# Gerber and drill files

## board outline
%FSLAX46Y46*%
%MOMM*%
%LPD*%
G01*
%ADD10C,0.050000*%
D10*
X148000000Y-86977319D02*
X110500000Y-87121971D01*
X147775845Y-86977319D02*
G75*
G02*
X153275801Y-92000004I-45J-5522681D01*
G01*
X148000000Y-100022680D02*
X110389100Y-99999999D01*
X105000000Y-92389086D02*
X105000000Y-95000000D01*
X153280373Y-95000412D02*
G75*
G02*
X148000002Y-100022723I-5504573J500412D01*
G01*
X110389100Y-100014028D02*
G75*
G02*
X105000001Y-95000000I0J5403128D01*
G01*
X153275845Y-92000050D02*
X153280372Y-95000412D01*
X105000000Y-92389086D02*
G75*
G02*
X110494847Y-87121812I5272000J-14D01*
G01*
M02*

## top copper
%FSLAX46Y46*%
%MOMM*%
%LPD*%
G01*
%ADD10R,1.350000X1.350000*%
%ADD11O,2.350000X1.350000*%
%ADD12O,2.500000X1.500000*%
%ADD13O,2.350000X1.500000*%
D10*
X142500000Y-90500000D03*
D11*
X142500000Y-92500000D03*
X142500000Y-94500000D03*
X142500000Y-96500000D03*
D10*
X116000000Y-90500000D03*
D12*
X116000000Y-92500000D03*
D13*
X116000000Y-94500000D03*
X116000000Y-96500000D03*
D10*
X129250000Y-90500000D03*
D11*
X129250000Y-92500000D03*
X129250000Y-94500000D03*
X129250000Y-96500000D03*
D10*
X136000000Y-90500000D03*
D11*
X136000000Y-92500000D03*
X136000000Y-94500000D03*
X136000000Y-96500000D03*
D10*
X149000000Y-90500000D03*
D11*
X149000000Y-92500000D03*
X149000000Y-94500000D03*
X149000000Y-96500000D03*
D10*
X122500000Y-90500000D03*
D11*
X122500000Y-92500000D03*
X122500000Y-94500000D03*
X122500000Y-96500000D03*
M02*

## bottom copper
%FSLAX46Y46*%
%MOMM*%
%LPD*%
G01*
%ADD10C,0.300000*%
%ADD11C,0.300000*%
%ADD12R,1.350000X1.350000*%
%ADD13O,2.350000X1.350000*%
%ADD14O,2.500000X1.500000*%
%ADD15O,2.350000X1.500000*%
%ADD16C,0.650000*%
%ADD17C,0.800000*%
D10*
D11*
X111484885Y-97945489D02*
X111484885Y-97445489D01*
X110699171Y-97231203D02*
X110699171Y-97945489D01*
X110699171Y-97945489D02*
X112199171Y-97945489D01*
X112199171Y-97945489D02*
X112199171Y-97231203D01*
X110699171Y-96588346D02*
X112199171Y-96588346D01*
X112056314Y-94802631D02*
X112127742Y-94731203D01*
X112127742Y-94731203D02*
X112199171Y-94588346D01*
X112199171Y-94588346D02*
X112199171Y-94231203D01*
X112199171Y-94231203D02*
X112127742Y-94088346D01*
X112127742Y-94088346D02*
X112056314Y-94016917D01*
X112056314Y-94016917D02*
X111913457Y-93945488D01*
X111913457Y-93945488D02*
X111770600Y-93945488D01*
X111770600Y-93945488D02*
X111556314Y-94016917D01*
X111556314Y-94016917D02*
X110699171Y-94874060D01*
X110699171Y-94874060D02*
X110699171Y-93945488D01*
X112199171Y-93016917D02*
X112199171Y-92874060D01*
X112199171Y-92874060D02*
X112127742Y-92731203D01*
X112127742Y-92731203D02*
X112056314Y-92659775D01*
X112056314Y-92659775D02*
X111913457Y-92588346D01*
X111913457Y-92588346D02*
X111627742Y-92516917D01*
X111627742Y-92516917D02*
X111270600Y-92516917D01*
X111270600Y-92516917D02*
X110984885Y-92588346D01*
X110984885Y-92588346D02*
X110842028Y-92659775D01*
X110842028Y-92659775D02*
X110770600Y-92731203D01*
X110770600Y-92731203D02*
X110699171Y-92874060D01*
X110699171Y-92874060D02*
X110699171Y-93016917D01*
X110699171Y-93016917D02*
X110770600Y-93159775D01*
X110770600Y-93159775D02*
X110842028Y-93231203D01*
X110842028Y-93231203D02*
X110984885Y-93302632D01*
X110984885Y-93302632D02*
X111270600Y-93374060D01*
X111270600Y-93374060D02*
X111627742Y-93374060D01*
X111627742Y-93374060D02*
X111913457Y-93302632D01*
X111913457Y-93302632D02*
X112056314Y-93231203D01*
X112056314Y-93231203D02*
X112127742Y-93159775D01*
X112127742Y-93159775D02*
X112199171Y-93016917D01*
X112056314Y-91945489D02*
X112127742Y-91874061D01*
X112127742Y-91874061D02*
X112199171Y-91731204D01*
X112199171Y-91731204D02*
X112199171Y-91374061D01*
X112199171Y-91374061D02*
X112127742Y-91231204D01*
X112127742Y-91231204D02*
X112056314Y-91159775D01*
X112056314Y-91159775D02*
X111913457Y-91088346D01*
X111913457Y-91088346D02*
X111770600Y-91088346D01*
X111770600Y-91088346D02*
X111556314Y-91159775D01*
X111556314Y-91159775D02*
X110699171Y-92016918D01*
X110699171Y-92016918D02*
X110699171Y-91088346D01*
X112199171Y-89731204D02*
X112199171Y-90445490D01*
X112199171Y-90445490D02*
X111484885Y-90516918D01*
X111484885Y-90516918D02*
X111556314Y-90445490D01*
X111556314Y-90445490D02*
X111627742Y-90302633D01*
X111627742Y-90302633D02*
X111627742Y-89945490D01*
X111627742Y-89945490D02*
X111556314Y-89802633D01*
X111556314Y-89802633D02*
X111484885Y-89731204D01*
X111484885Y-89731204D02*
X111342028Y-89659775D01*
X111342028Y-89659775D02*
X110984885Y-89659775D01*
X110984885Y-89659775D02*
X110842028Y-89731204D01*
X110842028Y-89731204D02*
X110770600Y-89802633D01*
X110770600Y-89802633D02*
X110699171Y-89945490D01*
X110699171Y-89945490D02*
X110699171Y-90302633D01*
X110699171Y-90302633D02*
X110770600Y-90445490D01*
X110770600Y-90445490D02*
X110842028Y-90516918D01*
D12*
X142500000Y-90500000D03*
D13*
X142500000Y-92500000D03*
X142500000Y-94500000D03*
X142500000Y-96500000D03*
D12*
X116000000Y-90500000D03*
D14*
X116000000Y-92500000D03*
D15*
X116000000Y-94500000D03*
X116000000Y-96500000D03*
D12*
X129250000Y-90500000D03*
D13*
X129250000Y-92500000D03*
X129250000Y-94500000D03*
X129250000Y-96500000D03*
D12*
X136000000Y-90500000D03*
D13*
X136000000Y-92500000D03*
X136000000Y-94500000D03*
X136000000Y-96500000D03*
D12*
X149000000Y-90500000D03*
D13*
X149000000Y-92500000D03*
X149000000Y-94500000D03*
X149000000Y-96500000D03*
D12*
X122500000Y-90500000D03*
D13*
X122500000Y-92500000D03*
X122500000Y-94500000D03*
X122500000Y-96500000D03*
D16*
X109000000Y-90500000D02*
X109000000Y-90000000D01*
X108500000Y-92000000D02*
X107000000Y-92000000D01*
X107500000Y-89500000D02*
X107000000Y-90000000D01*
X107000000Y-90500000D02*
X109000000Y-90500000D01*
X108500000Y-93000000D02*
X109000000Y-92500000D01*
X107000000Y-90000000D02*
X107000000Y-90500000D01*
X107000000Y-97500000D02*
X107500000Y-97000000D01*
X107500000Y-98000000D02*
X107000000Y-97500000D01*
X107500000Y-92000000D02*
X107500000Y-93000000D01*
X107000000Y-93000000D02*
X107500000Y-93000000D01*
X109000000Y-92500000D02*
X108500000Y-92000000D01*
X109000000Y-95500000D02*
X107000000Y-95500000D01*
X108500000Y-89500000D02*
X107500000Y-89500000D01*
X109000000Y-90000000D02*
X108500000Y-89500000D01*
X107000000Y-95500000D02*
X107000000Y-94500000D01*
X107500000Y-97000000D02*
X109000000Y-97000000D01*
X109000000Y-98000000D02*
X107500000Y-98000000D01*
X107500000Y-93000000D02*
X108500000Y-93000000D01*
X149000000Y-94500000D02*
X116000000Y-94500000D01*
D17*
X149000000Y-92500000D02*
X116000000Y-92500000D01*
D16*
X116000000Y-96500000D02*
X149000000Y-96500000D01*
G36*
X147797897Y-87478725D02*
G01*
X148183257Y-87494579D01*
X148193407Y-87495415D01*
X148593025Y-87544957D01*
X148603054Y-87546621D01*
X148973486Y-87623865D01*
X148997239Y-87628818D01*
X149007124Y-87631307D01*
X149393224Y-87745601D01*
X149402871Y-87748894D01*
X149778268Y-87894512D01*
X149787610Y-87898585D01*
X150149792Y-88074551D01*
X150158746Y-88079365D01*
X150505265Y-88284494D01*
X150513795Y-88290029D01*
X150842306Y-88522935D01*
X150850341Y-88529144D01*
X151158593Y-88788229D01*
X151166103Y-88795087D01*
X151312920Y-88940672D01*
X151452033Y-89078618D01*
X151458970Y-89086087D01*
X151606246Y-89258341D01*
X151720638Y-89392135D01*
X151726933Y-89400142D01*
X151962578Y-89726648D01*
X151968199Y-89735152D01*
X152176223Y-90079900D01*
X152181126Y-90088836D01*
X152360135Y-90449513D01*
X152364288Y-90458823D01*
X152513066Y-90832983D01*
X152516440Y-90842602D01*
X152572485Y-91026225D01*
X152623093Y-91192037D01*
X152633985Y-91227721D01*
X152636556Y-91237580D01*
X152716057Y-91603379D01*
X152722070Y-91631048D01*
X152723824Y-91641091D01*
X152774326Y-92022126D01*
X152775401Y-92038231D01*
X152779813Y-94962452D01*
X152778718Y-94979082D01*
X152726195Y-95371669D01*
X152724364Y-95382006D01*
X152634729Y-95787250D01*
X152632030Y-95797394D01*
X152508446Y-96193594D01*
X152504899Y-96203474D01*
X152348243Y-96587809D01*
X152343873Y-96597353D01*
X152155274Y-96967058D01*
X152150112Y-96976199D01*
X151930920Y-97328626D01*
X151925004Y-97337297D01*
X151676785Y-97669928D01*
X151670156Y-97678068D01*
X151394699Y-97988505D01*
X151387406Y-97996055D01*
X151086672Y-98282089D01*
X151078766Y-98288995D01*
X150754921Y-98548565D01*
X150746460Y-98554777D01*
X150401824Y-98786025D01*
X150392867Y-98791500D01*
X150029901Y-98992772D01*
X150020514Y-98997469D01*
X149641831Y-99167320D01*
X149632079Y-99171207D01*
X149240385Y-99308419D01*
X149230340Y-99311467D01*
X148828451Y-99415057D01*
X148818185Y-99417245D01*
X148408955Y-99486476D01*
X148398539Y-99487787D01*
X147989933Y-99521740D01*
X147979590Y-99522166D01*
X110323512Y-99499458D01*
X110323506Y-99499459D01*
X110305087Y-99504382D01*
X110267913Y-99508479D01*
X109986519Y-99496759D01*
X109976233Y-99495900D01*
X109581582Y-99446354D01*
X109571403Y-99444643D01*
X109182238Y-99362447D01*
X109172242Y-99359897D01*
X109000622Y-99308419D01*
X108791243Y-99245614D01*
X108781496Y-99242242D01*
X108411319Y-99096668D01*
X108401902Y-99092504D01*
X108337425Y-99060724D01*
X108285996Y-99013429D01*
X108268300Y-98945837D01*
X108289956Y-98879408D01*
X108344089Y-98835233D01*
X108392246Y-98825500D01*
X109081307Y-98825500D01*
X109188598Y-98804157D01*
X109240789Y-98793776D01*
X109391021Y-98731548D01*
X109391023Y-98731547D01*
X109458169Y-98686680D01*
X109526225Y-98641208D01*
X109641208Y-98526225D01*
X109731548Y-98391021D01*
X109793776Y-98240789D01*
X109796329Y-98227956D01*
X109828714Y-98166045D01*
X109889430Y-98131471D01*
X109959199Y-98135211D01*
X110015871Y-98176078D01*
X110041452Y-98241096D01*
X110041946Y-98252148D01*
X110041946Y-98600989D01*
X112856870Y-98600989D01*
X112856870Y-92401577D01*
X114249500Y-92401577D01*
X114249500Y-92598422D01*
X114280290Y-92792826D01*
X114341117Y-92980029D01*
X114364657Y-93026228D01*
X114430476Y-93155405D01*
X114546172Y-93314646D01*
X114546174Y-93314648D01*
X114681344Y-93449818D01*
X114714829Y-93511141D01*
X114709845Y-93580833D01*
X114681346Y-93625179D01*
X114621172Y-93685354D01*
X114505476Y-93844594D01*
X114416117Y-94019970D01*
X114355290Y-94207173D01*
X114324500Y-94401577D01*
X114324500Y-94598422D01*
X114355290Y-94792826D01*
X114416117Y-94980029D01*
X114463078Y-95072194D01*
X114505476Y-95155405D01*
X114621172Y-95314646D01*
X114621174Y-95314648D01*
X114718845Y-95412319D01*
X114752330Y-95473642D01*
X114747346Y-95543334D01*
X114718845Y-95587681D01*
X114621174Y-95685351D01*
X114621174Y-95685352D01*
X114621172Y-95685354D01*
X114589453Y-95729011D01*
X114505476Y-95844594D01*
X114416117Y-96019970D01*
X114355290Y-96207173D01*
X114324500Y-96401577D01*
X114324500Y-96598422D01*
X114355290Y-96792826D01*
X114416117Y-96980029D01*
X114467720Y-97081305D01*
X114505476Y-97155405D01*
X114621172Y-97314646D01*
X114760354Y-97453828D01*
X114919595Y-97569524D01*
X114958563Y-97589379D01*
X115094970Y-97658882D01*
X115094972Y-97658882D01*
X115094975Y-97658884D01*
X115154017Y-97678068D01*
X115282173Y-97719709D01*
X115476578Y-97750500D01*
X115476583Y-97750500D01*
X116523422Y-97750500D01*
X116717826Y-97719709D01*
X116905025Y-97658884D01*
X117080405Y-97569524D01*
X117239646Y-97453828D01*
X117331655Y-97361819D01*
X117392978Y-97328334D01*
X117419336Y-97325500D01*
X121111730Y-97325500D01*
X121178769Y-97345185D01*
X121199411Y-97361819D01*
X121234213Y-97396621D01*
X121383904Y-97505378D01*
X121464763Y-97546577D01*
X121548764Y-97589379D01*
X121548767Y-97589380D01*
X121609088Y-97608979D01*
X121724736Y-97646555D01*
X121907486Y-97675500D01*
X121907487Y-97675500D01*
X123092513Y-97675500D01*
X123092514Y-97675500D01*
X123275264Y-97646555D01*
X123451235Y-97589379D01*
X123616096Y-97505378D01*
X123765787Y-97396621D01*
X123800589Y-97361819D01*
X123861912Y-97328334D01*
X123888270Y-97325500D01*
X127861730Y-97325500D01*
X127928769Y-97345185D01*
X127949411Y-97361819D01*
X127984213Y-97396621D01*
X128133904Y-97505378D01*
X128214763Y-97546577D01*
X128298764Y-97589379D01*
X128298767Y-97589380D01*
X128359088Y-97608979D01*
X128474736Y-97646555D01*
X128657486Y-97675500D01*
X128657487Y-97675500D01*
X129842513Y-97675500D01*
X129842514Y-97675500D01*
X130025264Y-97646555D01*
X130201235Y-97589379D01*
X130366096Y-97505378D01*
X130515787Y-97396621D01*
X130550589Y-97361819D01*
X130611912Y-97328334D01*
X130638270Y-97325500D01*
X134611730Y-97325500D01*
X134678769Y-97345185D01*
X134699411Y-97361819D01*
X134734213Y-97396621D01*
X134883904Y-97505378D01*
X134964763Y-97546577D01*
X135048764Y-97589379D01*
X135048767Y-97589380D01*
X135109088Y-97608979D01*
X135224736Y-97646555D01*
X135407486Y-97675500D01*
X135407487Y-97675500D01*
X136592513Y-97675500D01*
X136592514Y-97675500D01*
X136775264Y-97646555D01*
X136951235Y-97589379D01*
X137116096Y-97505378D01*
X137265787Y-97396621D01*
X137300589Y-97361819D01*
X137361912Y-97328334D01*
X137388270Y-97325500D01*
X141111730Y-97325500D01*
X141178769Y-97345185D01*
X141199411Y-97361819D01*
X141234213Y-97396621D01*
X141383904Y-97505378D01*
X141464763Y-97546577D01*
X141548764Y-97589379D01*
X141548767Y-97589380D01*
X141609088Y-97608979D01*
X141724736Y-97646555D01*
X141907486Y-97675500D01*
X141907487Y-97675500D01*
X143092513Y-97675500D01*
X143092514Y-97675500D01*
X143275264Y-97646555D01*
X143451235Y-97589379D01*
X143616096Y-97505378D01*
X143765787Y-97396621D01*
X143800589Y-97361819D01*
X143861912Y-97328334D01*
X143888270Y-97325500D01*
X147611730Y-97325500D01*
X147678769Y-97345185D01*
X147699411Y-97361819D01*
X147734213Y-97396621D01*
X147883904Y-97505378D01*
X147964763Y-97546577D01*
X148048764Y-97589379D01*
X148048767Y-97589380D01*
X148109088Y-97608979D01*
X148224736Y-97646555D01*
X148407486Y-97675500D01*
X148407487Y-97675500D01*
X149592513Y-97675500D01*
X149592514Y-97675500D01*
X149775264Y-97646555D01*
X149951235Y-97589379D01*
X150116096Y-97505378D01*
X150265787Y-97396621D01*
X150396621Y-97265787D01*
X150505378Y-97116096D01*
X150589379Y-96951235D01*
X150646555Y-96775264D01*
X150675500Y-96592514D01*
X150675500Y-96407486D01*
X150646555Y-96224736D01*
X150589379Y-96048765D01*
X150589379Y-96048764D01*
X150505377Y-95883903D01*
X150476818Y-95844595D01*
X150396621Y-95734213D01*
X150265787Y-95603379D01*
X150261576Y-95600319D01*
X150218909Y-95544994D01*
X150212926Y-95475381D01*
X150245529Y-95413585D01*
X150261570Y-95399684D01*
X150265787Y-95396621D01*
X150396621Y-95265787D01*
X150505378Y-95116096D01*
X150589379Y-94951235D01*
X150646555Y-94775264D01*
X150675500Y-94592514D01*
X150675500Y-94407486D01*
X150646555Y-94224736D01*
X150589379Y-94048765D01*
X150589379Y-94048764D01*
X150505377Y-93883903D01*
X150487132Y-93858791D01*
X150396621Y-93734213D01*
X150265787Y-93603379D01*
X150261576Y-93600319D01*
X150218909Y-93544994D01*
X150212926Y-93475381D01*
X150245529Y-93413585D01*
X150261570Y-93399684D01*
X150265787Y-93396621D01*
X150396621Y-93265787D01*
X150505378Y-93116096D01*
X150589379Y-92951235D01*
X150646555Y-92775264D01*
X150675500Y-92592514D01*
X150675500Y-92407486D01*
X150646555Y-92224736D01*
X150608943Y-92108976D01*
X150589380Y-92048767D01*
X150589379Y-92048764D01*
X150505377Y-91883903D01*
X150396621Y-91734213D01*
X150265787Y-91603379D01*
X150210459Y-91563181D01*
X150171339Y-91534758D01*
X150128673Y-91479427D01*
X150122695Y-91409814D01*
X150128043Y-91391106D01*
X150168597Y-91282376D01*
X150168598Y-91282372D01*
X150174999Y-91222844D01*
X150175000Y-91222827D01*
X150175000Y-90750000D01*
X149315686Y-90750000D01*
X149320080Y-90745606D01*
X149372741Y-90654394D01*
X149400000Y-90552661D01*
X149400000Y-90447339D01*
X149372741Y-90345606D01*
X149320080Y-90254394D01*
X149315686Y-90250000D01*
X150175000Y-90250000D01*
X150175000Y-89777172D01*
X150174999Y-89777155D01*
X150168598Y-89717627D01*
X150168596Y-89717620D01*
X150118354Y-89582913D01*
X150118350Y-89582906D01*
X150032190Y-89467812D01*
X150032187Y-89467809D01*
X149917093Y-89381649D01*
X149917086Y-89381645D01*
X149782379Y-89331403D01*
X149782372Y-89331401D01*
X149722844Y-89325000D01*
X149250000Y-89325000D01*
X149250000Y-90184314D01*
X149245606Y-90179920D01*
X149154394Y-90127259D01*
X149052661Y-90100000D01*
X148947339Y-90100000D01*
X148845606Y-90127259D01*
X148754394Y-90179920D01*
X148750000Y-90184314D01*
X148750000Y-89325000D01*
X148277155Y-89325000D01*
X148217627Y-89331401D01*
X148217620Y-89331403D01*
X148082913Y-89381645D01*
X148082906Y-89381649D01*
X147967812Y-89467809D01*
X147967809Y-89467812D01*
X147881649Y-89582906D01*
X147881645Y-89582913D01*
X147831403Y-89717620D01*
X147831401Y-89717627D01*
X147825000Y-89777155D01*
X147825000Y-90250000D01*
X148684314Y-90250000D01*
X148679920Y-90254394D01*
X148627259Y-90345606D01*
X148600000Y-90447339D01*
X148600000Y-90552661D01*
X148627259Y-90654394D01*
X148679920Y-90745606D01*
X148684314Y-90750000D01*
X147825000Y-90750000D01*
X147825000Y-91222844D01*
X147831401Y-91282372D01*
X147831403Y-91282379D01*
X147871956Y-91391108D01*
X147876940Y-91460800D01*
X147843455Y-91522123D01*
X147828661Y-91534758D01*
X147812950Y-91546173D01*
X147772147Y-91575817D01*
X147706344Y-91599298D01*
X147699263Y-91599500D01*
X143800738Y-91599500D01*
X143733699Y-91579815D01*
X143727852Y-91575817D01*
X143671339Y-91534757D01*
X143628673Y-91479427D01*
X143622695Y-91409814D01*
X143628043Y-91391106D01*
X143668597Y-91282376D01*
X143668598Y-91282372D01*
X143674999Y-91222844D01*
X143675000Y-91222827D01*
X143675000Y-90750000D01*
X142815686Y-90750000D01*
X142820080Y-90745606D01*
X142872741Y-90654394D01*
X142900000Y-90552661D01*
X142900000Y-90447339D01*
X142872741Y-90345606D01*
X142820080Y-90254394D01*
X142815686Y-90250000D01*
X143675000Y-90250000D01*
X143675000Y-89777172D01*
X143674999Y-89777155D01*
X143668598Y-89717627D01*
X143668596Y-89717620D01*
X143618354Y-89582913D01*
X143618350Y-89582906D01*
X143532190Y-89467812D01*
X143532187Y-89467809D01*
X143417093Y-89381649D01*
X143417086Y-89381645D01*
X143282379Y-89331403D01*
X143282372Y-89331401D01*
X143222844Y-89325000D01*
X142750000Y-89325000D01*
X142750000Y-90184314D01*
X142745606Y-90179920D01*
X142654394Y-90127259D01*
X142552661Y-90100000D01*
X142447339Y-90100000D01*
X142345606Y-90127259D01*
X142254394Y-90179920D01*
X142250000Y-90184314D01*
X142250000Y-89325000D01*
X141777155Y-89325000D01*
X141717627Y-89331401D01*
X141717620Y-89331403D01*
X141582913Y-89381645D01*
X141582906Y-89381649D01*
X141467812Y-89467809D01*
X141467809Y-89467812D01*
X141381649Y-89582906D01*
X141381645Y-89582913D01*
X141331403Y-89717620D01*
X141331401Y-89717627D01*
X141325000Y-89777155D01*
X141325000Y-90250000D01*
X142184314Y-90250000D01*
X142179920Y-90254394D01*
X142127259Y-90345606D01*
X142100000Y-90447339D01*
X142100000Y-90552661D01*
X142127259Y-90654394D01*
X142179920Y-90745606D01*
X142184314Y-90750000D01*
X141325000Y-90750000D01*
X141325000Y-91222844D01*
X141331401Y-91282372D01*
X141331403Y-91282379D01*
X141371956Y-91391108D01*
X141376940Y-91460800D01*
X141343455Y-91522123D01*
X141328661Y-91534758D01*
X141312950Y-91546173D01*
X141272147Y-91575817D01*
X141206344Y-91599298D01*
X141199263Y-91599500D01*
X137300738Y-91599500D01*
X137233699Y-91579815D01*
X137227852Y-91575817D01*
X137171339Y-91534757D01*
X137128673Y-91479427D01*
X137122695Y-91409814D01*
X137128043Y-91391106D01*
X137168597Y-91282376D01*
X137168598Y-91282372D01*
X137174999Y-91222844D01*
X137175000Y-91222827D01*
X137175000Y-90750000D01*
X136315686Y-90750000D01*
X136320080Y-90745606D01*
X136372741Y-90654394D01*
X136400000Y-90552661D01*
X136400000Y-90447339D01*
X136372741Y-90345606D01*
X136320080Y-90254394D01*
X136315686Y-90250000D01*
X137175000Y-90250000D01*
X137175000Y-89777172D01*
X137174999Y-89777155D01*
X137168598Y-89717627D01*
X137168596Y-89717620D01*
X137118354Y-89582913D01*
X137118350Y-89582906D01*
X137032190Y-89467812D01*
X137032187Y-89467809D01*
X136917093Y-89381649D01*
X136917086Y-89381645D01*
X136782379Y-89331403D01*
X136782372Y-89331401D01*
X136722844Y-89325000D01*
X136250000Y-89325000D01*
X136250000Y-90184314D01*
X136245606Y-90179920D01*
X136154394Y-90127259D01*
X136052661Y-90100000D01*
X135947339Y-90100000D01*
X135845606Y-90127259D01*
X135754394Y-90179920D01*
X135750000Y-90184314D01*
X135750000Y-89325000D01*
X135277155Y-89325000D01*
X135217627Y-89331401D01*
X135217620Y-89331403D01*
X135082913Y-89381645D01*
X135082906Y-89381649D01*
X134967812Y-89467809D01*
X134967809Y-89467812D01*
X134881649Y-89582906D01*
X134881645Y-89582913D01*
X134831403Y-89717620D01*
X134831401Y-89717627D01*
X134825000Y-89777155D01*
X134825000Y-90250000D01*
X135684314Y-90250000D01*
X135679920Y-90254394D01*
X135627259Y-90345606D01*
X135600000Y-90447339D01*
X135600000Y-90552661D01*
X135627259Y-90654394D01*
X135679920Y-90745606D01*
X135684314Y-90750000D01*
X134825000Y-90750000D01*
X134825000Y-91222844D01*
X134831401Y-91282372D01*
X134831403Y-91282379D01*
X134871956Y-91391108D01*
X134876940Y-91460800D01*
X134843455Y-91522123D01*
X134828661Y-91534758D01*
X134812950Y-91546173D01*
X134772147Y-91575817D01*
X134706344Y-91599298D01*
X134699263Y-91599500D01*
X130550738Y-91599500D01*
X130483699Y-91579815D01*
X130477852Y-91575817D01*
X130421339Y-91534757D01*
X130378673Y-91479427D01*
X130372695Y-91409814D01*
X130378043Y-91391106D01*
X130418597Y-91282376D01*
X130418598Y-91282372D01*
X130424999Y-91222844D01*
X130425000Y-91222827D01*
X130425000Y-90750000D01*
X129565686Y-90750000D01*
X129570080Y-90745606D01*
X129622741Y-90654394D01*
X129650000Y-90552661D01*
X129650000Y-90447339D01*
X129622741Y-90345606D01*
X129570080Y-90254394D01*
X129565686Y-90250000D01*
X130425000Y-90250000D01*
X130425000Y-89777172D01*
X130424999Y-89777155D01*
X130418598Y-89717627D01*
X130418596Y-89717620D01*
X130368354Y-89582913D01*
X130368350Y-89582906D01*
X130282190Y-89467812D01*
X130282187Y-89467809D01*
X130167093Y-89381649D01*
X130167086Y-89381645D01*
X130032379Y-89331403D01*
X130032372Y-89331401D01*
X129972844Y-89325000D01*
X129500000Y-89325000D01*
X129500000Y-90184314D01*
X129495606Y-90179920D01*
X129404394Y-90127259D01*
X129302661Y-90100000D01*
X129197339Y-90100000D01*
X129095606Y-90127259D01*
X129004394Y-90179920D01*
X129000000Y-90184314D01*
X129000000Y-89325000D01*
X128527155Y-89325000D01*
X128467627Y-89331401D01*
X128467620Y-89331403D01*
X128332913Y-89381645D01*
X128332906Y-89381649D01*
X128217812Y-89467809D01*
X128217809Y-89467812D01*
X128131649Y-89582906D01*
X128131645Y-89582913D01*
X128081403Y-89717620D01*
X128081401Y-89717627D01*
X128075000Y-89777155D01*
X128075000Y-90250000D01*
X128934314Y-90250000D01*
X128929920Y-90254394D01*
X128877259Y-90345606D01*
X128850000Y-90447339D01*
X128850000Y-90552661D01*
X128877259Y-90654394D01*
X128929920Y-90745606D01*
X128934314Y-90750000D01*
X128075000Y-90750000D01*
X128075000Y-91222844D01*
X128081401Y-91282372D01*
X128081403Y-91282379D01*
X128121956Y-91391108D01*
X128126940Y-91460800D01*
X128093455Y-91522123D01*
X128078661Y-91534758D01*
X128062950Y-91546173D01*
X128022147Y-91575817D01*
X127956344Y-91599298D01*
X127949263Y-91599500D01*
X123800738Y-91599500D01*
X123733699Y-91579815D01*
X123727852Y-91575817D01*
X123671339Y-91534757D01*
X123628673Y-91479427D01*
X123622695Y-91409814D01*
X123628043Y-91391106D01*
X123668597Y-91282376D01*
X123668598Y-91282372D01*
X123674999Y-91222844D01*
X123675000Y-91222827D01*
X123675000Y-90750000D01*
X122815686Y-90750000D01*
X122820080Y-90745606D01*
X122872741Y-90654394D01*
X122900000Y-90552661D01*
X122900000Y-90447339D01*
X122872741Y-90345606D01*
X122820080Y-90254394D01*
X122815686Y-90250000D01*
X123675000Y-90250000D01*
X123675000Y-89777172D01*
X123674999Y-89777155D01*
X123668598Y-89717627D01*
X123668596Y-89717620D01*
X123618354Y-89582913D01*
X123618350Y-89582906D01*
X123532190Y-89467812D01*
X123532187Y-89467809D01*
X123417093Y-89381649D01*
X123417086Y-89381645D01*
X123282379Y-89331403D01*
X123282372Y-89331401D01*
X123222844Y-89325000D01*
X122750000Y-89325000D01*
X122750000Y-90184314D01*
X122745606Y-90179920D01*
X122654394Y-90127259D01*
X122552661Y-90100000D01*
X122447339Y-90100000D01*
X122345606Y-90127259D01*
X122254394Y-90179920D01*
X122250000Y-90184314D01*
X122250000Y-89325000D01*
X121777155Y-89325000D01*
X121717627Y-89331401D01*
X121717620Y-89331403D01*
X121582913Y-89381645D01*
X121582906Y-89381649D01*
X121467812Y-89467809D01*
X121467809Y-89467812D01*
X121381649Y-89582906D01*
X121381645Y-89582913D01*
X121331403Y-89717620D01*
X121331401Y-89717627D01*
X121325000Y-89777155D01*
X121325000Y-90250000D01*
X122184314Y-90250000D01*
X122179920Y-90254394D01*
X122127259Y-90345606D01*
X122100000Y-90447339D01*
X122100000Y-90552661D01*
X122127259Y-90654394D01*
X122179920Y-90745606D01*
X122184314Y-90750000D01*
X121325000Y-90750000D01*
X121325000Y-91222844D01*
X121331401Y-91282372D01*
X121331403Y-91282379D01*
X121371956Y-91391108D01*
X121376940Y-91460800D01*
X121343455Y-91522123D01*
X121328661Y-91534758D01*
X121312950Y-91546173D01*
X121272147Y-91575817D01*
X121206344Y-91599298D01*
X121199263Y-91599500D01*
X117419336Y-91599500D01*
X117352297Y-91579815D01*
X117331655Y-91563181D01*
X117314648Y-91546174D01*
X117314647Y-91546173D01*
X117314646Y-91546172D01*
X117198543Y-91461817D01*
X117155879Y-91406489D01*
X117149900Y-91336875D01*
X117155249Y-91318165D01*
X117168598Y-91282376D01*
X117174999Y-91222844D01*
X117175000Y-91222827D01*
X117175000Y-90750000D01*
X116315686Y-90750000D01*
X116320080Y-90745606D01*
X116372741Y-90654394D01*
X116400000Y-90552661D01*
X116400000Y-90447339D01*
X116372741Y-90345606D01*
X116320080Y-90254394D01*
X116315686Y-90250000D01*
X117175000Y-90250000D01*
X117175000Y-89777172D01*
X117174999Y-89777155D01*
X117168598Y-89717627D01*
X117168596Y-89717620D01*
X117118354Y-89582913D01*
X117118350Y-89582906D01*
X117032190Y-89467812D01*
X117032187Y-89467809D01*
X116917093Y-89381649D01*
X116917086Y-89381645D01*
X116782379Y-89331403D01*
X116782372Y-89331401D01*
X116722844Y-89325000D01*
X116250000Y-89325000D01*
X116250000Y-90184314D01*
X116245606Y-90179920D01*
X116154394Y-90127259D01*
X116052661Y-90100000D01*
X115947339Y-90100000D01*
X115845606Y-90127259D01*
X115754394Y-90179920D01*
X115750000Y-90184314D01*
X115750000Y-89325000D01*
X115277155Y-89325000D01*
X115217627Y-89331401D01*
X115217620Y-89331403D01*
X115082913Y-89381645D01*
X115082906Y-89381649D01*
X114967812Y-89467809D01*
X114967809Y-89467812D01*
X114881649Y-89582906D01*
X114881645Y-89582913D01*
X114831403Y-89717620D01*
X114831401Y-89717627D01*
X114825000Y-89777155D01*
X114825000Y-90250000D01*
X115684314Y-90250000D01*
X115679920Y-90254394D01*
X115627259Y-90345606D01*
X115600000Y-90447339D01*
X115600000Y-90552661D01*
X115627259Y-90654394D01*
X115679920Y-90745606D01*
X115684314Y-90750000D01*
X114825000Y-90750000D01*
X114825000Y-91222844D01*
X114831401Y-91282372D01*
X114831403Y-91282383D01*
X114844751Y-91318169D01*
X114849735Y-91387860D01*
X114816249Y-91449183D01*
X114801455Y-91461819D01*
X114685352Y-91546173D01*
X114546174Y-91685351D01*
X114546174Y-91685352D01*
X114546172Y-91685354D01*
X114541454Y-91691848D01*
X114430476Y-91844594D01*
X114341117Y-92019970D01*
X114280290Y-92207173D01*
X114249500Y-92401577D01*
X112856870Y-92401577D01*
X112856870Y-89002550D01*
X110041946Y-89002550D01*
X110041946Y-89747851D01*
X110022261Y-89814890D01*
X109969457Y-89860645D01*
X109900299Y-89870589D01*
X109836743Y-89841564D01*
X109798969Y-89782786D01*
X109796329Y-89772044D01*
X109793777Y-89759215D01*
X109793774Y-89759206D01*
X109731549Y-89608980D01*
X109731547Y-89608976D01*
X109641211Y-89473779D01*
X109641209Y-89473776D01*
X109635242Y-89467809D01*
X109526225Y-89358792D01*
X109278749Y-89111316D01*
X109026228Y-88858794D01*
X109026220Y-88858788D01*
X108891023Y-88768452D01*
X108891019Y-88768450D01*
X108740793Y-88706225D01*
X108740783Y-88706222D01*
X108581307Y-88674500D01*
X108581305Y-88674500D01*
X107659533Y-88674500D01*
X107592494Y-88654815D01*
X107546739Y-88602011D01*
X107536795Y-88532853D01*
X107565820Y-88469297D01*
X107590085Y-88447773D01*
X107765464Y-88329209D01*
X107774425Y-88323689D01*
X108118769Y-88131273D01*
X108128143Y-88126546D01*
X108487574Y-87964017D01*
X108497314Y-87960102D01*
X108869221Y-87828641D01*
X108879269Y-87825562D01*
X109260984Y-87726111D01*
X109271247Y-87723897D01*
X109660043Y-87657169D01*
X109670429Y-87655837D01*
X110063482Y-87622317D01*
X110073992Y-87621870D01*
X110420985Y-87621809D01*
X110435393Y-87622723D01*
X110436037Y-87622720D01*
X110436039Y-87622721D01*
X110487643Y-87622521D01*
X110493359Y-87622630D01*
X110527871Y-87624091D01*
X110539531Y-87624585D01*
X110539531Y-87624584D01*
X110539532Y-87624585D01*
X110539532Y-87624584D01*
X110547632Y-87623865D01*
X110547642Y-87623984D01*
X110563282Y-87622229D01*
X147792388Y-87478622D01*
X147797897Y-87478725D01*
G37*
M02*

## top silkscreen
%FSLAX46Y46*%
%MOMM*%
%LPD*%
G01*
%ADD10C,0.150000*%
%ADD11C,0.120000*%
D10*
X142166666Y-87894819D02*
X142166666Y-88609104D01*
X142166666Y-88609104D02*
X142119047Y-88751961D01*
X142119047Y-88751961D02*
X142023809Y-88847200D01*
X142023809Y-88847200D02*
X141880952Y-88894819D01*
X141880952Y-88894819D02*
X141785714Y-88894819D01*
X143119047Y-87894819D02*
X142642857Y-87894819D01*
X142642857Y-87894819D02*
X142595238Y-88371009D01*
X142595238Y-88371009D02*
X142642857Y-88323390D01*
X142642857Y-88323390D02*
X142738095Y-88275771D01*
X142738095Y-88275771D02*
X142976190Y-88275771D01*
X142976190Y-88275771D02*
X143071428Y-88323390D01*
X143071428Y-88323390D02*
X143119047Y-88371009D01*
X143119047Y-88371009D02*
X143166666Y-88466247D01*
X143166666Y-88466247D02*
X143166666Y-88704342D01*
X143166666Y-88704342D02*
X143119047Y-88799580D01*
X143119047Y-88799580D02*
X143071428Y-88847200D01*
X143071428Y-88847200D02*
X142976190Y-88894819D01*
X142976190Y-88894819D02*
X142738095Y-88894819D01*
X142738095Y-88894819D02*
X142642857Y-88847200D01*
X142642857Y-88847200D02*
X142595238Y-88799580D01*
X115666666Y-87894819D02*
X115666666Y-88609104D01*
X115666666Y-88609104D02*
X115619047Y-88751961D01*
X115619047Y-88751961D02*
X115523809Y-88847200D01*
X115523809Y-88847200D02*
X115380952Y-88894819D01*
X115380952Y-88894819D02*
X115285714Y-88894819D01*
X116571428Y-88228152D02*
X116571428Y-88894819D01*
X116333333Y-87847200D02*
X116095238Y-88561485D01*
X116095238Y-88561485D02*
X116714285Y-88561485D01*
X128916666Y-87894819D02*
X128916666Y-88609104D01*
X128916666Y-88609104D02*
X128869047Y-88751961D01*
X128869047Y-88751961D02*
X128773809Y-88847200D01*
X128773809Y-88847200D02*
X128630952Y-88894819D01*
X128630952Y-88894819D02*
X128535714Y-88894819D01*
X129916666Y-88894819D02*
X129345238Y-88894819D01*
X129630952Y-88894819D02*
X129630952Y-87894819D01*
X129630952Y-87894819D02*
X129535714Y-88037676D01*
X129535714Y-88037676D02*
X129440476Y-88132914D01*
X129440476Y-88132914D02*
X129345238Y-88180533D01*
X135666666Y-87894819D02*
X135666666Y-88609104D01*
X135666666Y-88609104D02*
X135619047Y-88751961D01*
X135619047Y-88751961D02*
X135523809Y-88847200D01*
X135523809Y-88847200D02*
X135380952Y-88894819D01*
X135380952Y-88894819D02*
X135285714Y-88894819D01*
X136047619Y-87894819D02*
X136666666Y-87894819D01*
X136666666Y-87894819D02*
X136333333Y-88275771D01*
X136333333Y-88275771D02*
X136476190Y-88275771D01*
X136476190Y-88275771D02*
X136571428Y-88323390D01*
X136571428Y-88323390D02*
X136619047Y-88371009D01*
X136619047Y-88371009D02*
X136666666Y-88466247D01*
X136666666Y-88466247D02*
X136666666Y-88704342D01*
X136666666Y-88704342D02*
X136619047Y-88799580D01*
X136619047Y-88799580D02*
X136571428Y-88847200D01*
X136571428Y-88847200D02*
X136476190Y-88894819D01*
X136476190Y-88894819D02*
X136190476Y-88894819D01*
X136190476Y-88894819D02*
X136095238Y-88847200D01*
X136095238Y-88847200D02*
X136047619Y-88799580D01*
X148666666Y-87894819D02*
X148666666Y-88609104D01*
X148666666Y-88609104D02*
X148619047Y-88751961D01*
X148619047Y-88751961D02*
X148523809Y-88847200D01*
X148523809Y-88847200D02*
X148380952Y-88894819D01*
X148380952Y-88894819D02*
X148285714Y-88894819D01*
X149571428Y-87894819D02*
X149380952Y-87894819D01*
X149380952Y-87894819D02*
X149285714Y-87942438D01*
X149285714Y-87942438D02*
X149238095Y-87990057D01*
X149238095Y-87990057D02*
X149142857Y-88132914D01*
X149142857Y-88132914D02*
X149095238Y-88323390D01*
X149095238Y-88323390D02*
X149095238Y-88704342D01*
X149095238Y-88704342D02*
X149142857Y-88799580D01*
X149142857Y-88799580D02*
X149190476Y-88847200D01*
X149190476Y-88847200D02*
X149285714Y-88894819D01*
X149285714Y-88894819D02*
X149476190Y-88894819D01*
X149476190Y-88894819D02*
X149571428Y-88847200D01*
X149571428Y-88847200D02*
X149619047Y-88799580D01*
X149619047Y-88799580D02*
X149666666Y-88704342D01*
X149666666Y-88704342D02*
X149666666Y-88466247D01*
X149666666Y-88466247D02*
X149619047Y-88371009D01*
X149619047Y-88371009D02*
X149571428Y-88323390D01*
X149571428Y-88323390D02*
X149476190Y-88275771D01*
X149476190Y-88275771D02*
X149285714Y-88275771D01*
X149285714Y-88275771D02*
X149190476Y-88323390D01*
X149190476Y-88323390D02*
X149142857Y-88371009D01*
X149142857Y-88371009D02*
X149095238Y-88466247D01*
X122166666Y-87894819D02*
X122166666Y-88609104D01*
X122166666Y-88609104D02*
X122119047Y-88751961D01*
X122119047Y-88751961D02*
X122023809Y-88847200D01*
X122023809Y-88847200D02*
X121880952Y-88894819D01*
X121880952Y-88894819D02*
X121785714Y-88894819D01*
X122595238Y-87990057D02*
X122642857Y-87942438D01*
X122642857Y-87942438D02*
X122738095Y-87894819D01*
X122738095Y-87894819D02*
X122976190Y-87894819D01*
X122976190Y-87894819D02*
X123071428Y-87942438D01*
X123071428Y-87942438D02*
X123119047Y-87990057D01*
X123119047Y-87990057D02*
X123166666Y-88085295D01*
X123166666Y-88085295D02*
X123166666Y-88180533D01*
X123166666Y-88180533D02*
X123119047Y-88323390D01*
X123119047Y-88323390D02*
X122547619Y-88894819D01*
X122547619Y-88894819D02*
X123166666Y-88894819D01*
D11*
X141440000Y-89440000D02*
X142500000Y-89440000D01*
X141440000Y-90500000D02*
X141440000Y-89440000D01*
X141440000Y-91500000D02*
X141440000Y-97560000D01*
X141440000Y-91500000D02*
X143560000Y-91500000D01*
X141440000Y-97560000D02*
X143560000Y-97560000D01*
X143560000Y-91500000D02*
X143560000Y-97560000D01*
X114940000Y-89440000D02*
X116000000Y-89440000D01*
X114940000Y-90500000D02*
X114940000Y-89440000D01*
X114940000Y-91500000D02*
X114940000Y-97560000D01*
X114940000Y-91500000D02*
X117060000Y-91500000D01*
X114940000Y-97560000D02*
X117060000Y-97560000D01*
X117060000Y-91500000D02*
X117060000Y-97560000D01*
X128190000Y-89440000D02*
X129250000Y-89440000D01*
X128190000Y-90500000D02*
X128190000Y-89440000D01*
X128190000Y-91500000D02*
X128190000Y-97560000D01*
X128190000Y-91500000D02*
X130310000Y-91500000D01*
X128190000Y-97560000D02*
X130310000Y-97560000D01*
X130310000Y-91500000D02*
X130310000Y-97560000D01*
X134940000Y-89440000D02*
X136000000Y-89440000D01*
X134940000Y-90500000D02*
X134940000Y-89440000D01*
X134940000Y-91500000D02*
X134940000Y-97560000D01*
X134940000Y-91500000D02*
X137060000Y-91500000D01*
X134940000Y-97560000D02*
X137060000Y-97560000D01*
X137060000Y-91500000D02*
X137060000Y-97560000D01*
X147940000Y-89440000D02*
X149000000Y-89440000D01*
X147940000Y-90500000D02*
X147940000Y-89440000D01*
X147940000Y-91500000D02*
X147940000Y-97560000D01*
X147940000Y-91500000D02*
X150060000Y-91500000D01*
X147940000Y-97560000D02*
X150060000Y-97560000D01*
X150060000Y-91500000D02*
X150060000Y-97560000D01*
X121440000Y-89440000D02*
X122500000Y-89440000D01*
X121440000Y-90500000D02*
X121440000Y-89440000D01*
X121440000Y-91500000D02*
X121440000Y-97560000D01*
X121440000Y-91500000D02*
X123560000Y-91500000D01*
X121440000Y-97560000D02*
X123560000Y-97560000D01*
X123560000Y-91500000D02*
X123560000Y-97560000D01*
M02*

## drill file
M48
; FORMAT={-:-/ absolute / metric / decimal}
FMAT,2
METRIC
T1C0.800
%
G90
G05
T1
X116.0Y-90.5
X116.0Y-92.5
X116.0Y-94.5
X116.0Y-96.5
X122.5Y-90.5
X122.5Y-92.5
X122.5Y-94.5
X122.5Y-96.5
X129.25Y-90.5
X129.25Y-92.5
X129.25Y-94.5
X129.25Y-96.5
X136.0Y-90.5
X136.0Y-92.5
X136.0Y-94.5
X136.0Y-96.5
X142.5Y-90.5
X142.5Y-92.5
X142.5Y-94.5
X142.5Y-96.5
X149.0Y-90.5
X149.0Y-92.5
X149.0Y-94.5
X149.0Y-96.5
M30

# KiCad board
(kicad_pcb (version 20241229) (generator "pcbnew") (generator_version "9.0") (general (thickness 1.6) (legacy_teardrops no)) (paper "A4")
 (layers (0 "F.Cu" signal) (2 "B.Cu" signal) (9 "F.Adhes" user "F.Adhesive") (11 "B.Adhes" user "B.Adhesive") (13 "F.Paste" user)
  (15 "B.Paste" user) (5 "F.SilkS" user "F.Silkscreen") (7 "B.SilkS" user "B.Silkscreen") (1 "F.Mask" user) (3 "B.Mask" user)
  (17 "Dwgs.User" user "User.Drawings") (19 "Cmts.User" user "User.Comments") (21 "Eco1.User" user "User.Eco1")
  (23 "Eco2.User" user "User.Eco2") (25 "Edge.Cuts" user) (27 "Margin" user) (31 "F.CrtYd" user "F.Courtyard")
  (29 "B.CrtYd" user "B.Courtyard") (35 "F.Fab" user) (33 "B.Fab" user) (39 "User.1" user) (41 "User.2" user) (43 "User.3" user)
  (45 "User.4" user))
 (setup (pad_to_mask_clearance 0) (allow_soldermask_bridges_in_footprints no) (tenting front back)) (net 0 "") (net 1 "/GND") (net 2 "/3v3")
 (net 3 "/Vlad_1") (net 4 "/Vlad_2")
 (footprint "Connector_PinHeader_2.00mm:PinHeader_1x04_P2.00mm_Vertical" (layer "F.Cu") (at 142.5 90.5)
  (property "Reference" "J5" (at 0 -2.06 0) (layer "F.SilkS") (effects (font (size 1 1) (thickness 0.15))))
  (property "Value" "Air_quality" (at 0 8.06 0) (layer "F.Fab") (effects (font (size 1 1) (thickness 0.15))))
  (fp_line (start -1.06 -1.06) (end 0 -1.06) (stroke (width 0.12) (type solid)) (layer "F.SilkS"))
  (fp_line (start -1.06 0) (end -1.06 -1.06) (stroke (width 0.12) (type solid)) (layer "F.SilkS"))
  (fp_line (start -1.06 1) (end -1.06 7.06) (stroke (width 0.12) (type solid)) (layer "F.SilkS"))
  (fp_line (start -1.06 1) (end 1.06 1) (stroke (width 0.12) (type solid)) (layer "F.SilkS"))
  (fp_line (start -1.06 7.06) (end 1.06 7.06) (stroke (width 0.12) (type solid)) (layer "F.SilkS"))
  (fp_line (start 1.06 1) (end 1.06 7.06) (stroke (width 0.12) (type solid)) (layer "F.SilkS"))
  (pad "1" thru_hole rect (at 0 0) (size 1.35 1.35) (drill 0.8) (layers "*.Cu" "*.Mask") (remove_unused_layers no) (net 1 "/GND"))
  (pad "2" thru_hole oval (at 0 2) (size 2.35 1.35) (drill 0.8) (layers "*.Cu" "*.Mask") (remove_unused_layers no) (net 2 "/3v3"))
  (pad "3" thru_hole oval (at 0 4) (size 2.35 1.35) (drill 0.8) (layers "*.Cu" "*.Mask") (remove_unused_layers no) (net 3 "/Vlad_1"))
  (pad "4" thru_hole oval (at 0 6) (size 2.35 1.35) (drill 0.8) (layers "*.Cu" "*.Mask") (remove_unused_layers no) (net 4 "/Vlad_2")))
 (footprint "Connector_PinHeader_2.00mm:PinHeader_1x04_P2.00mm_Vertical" (layer "F.Cu") (at 116 90.5)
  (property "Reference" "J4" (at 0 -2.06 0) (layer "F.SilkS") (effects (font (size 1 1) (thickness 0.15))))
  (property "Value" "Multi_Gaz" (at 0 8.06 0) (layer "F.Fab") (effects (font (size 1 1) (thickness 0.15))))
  (fp_line (start -1.06 -1.06) (end 0 -1.06) (stroke (width 0.12) (type solid)) (layer "F.SilkS"))
  (fp_line (start -1.06 0) (end -1.06 -1.06) (stroke (width 0.12) (type solid)) (layer "F.SilkS"))
  (fp_line (start -1.06 1) (end -1.06 7.06) (stroke (width 0.12) (type solid)) (layer "F.SilkS"))
  (fp_line (start -1.06 1) (end 1.06 1) (stroke (width 0.12) (type solid)) (layer "F.SilkS"))
  (fp_line (start -1.06 7.06) (end 1.06 7.06) (stroke (width 0.12) (type solid)) (layer "F.SilkS"))
  (fp_line (start 1.06 1) (end 1.06 7.06) (stroke (width 0.12) (type solid)) (layer "F.SilkS"))
  (pad "1" thru_hole rect (at 0 0) (size 1.35 1.35) (drill 0.8) (layers "*.Cu" "*.Mask") (remove_unused_layers no) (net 1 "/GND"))
  (pad "2" thru_hole oval (at 0 2) (size 2.5 1.5) (drill 0.8) (layers "*.Cu" "*.Mask") (remove_unused_layers no) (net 2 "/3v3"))
  (pad "3" thru_hole oval (at 0 4) (size 2.35 1.5) (drill 0.8) (layers "*.Cu" "*.Mask") (remove_unused_layers no) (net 3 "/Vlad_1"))
  (pad "4" thru_hole oval (at 0 6) (size 2.35 1.5) (drill 0.8) (layers "*.Cu" "*.Mask") (remove_unused_layers no) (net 4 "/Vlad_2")))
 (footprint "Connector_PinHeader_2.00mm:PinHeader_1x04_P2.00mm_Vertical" (layer "F.Cu") (at 129.25 90.5)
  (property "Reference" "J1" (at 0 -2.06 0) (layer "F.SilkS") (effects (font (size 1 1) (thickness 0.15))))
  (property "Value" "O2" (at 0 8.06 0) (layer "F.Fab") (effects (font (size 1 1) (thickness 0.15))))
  (fp_line (start -1.06 -1.06) (end 0 -1.06) (stroke (width 0.12) (type solid)) (layer "F.SilkS"))
  (fp_line (start -1.06 0) (end -1.06 -1.06) (stroke (width 0.12) (type solid)) (layer "F.SilkS"))
  (fp_line (start -1.06 1) (end -1.06 7.06) (stroke (width 0.12) (type solid)) (layer "F.SilkS"))
  (fp_line (start -1.06 1) (end 1.06 1) (stroke (width 0.12) (type solid)) (layer "F.SilkS"))
  (fp_line (start -1.06 7.06) (end 1.06 7.06) (stroke (width 0.12) (type solid)) (layer "F.SilkS"))
  (fp_line (start 1.06 1) (end 1.06 7.06) (stroke (width 0.12) (type solid)) (layer "F.SilkS"))
  (pad "1" thru_hole rect (at 0 0) (size 1.35 1.35) (drill 0.8) (layers "*.Cu" "*.Mask") (remove_unused_layers no) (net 1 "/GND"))
  (pad "2" thru_hole oval (at 0 2) (size 2.35 1.35) (drill 0.8) (layers "*.Cu" "*.Mask") (remove_unused_layers no) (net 2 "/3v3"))
  (pad "3" thru_hole oval (at 0 4) (size 2.35 1.35) (drill 0.8) (layers "*.Cu" "*.Mask") (remove_unused_layers no) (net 3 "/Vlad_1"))
  (pad "4" thru_hole oval (at 0 6) (size 2.35 1.35) (drill 0.8) (layers "*.Cu" "*.Mask") (remove_unused_layers no) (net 4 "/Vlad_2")))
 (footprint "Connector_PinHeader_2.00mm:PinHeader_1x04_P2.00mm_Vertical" (layer "F.Cu") (at 136 90.5)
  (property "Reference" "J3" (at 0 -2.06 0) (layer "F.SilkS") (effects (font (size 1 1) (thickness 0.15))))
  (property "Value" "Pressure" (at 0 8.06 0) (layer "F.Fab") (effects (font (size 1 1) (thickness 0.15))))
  (fp_line (start -1.06 -1.06) (end 0 -1.06) (stroke (width 0.12) (type solid)) (layer "F.SilkS"))
  (fp_line (start -1.06 0) (end -1.06 -1.06) (stroke (width 0.12) (type solid)) (layer "F.SilkS"))
  (fp_line (start -1.06 1) (end -1.06 7.06) (stroke (width 0.12) (type solid)) (layer "F.SilkS"))
  (fp_line (start -1.06 1) (end 1.06 1) (stroke (width 0.12) (type solid)) (layer "F.SilkS"))
  (fp_line (start -1.06 7.06) (end 1.06 7.06) (stroke (width 0.12) (type solid)) (layer "F.SilkS"))
  (fp_line (start 1.06 1) (end 1.06 7.06) (stroke (width 0.12) (type solid)) (layer "F.SilkS"))
  (pad "1" thru_hole rect (at 0 0) (size 1.35 1.35) (drill 0.8) (layers "*.Cu" "*.Mask") (remove_unused_layers no) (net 1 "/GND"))
  (pad "2" thru_hole oval (at 0 2) (size 2.35 1.35) (drill 0.8) (layers "*.Cu" "*.Mask") (remove_unused_layers no) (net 2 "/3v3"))
  (pad "3" thru_hole oval (at 0 4) (size 2.35 1.35) (drill 0.8) (layers "*.Cu" "*.Mask") (remove_unused_layers no) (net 3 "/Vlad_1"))
  (pad "4" thru_hole oval (at 0 6) (size 2.35 1.35) (drill 0.8) (layers "*.Cu" "*.Mask") (remove_unused_layers no) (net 4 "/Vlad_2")))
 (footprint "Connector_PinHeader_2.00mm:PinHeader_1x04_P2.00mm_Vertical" (layer "F.Cu") (at 149 90.5)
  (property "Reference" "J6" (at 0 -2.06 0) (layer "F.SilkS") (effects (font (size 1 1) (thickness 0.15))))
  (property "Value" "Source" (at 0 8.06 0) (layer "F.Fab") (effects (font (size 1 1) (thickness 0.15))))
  (fp_line (start -1.06 -1.06) (end 0 -1.06) (stroke (width 0.12) (type solid)) (layer "F.SilkS"))
  (fp_line (start -1.06 0) (end -1.06 -1.06) (stroke (width 0.12) (type solid)) (layer "F.SilkS"))
  (fp_line (start -1.06 1) (end -1.06 7.06) (stroke (width 0.12) (type solid)) (layer "F.SilkS"))
  (fp_line (start -1.06 1) (end 1.06 1) (stroke (width 0.12) (type solid)) (layer "F.SilkS"))
  (fp_line (start -1.06 7.06) (end 1.06 7.06) (stroke (width 0.12) (type solid)) (layer "F.SilkS"))
  (fp_line (start 1.06 1) (end 1.06 7.06) (stroke (width 0.12) (type solid)) (layer "F.SilkS"))
  (pad "1" thru_hole rect (at 0 0) (size 1.35 1.35) (drill 0.8) (layers "*.Cu" "*.Mask") (remove_unused_layers no) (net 1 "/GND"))
  (pad "2" thru_hole oval (at 0 2) (size 2.35 1.35) (drill 0.8) (layers "*.Cu" "F.Mask") (remove_unused_layers no) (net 2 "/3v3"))
  (pad "3" thru_hole oval (at 0 4) (size 2.35 1.35) (drill 0.8) (layers "*.Cu" "*.Mask") (remove_unused_layers no) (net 3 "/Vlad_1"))
  (pad "4" thru_hole oval (at 0 6) (size 2.35 1.35) (drill 0.8) (layers "*.Cu" "*.Mask") (remove_unused_layers no) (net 4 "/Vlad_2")))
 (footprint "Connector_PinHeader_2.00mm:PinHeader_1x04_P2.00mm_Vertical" (layer "F.Cu") (at 122.5 90.5)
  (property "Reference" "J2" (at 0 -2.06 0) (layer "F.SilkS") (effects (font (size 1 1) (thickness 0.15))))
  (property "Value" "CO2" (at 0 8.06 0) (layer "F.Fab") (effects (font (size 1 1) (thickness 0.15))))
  (fp_line (start -1.06 -1.06) (end 0 -1.06) (stroke (width 0.12) (type solid)) (layer "F.SilkS"))
  (fp_line (start -1.06 0) (end -1.06 -1.06) (stroke (width 0.12) (type solid)) (layer "F.SilkS"))
  (fp_line (start -1.06 1) (end -1.06 7.06) (stroke (width 0.12) (type solid)) (layer "F.SilkS"))
  (fp_line (start -1.06 1) (end 1.06 1) (stroke (width 0.12) (type solid)) (layer "F.SilkS"))
  (fp_line (start -1.06 7.06) (end 1.06 7.06) (stroke (width 0.12) (type solid)) (layer "F.SilkS"))
  (fp_line (start 1.06 1) (end 1.06 7.06) (stroke (width 0.12) (type solid)) (layer "F.SilkS"))
  (pad "1" thru_hole rect (at 0 0) (size 1.35 1.35) (drill 0.8) (layers "*.Cu" "*.Mask") (remove_unused_layers no) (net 1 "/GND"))
  (pad "2" thru_hole oval (at 0 2) (size 2.35 1.35) (drill 0.8) (layers "*.Cu" "*.Mask") (remove_unused_layers no) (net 2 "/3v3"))
  (pad "3" thru_hole oval (at 0 4) (size 2.35 1.35) (drill 0.8) (layers "*.Cu" "*.Mask") (remove_unused_layers no) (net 3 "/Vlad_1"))
  (pad "4" thru_hole oval (at 0 6) (size 2.35 1.35) (drill 0.8) (layers "*.Cu" "*.Mask") (remove_unused_layers no) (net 4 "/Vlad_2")))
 (gr_line (start 148 86.977319) (end 110.5 87.121971) (stroke (width 0.05) (type default)) (layer "Edge.Cuts"))
 (gr_arc (start 147.775845 86.977319) (mid 151.5 88.421928) (end 153.275845 92) (stroke (width 0.05) (type default)) (layer "Edge.Cuts"))
 (gr_line (start 148 100.02268) (end 110.3891 99.999999) (stroke (width 0.05) (type default)) (layer "Edge.Cuts"))
 (gr_line (start 105 92.389086) (end 105 95) (stroke (width 0.05) (type default)) (layer "Edge.Cuts"))
 (gr_arc (start 153.280373 95.000412) (mid 151.585077 98.504996) (end 148 100.02268) (stroke (width 0.05) (type default))
  (layer "Edge.Cuts"))
 (gr_arc (start 110.3891 100.014028) (mid 106.708645 98.566669) (end 105 95) (stroke (width 0.05) (type default)) (layer "Edge.Cuts"))
 (gr_line (start 153.275845 92.00005) (end 153.280372 95.000412) (stroke (width 0.05) (type default)) (layer "Edge.Cuts"))
 (gr_arc (start 105 92.389086) (mid 106.62377 88.583227) (end 110.49485 87.121747) (stroke (width 0.05) (type default)) (layer "Edge.Cuts"))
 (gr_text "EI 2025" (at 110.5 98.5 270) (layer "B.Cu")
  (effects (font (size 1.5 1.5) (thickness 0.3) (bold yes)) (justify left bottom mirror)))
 (segment (start 109 90.5) (end 109 90) (width 0.65) (layer "B.Cu") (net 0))
 (segment (start 108.5 92) (end 107 92) (width 0.65) (layer "B.Cu") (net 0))
 (segment (start 107.5 89.5) (end 107 90) (width 0.65) (layer "B.Cu") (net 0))
 (segment (start 107 90.5) (end 109 90.5) (width 0.65) (layer "B.Cu") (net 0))
 (segment (start 108.5 93) (end 109 92.5) (width 0.65) (layer "B.Cu") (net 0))
 (segment (start 107 90) (end 107 90.5) (width 0.65) (layer "B.Cu") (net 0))
 (segment (start 107 97.5) (end 107.5 97) (width 0.65) (layer "B.Cu") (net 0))
 (segment (start 107.5 98) (end 107 97.5) (width 0.65) (layer "B.Cu") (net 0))
 (segment (start 107.5 92) (end 107.5 93) (width 0.65) (layer "B.Cu") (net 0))
 (segment (start 107 93) (end 107.5 93) (width 0.65) (layer "B.Cu") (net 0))
 (segment (start 109 92.5) (end 108.5 92) (width 0.65) (layer "B.Cu") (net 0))
 (segment (start 109 95.5) (end 107 95.5) (width 0.65) (layer "B.Cu") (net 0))
 (segment (start 108.5 89.5) (end 107.5 89.5) (width 0.65) (layer "B.Cu") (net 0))
 (segment (start 109 90) (end 108.5 89.5) (width 0.65) (layer "B.Cu") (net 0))
 (segment (start 107 95.5) (end 107 94.5) (width 0.65) (layer "B.Cu") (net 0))
 (segment (start 107.5 97) (end 109 97) (width 0.65) (layer "B.Cu") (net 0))
 (segment (start 109 98) (end 107.5 98) (width 0.65) (layer "B.Cu") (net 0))
 (segment (start 107.5 93) (end 108.5 93) (width 0.65) (layer "B.Cu") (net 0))
 (segment (start 149 94.5) (end 116 94.5) (width 0.65) (layer "B.Cu") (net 3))
 (segment (start 149 92.5) (end 116 92.5) (width 0.8) (layer "B.Cu") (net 2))
 (segment (start 116 96.5) (end 149 96.5) (width 0.65) (layer "B.Cu") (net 4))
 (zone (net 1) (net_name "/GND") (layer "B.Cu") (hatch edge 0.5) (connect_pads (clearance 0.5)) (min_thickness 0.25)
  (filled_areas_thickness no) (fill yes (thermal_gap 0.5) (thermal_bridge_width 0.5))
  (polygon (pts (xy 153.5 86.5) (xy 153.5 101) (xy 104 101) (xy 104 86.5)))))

